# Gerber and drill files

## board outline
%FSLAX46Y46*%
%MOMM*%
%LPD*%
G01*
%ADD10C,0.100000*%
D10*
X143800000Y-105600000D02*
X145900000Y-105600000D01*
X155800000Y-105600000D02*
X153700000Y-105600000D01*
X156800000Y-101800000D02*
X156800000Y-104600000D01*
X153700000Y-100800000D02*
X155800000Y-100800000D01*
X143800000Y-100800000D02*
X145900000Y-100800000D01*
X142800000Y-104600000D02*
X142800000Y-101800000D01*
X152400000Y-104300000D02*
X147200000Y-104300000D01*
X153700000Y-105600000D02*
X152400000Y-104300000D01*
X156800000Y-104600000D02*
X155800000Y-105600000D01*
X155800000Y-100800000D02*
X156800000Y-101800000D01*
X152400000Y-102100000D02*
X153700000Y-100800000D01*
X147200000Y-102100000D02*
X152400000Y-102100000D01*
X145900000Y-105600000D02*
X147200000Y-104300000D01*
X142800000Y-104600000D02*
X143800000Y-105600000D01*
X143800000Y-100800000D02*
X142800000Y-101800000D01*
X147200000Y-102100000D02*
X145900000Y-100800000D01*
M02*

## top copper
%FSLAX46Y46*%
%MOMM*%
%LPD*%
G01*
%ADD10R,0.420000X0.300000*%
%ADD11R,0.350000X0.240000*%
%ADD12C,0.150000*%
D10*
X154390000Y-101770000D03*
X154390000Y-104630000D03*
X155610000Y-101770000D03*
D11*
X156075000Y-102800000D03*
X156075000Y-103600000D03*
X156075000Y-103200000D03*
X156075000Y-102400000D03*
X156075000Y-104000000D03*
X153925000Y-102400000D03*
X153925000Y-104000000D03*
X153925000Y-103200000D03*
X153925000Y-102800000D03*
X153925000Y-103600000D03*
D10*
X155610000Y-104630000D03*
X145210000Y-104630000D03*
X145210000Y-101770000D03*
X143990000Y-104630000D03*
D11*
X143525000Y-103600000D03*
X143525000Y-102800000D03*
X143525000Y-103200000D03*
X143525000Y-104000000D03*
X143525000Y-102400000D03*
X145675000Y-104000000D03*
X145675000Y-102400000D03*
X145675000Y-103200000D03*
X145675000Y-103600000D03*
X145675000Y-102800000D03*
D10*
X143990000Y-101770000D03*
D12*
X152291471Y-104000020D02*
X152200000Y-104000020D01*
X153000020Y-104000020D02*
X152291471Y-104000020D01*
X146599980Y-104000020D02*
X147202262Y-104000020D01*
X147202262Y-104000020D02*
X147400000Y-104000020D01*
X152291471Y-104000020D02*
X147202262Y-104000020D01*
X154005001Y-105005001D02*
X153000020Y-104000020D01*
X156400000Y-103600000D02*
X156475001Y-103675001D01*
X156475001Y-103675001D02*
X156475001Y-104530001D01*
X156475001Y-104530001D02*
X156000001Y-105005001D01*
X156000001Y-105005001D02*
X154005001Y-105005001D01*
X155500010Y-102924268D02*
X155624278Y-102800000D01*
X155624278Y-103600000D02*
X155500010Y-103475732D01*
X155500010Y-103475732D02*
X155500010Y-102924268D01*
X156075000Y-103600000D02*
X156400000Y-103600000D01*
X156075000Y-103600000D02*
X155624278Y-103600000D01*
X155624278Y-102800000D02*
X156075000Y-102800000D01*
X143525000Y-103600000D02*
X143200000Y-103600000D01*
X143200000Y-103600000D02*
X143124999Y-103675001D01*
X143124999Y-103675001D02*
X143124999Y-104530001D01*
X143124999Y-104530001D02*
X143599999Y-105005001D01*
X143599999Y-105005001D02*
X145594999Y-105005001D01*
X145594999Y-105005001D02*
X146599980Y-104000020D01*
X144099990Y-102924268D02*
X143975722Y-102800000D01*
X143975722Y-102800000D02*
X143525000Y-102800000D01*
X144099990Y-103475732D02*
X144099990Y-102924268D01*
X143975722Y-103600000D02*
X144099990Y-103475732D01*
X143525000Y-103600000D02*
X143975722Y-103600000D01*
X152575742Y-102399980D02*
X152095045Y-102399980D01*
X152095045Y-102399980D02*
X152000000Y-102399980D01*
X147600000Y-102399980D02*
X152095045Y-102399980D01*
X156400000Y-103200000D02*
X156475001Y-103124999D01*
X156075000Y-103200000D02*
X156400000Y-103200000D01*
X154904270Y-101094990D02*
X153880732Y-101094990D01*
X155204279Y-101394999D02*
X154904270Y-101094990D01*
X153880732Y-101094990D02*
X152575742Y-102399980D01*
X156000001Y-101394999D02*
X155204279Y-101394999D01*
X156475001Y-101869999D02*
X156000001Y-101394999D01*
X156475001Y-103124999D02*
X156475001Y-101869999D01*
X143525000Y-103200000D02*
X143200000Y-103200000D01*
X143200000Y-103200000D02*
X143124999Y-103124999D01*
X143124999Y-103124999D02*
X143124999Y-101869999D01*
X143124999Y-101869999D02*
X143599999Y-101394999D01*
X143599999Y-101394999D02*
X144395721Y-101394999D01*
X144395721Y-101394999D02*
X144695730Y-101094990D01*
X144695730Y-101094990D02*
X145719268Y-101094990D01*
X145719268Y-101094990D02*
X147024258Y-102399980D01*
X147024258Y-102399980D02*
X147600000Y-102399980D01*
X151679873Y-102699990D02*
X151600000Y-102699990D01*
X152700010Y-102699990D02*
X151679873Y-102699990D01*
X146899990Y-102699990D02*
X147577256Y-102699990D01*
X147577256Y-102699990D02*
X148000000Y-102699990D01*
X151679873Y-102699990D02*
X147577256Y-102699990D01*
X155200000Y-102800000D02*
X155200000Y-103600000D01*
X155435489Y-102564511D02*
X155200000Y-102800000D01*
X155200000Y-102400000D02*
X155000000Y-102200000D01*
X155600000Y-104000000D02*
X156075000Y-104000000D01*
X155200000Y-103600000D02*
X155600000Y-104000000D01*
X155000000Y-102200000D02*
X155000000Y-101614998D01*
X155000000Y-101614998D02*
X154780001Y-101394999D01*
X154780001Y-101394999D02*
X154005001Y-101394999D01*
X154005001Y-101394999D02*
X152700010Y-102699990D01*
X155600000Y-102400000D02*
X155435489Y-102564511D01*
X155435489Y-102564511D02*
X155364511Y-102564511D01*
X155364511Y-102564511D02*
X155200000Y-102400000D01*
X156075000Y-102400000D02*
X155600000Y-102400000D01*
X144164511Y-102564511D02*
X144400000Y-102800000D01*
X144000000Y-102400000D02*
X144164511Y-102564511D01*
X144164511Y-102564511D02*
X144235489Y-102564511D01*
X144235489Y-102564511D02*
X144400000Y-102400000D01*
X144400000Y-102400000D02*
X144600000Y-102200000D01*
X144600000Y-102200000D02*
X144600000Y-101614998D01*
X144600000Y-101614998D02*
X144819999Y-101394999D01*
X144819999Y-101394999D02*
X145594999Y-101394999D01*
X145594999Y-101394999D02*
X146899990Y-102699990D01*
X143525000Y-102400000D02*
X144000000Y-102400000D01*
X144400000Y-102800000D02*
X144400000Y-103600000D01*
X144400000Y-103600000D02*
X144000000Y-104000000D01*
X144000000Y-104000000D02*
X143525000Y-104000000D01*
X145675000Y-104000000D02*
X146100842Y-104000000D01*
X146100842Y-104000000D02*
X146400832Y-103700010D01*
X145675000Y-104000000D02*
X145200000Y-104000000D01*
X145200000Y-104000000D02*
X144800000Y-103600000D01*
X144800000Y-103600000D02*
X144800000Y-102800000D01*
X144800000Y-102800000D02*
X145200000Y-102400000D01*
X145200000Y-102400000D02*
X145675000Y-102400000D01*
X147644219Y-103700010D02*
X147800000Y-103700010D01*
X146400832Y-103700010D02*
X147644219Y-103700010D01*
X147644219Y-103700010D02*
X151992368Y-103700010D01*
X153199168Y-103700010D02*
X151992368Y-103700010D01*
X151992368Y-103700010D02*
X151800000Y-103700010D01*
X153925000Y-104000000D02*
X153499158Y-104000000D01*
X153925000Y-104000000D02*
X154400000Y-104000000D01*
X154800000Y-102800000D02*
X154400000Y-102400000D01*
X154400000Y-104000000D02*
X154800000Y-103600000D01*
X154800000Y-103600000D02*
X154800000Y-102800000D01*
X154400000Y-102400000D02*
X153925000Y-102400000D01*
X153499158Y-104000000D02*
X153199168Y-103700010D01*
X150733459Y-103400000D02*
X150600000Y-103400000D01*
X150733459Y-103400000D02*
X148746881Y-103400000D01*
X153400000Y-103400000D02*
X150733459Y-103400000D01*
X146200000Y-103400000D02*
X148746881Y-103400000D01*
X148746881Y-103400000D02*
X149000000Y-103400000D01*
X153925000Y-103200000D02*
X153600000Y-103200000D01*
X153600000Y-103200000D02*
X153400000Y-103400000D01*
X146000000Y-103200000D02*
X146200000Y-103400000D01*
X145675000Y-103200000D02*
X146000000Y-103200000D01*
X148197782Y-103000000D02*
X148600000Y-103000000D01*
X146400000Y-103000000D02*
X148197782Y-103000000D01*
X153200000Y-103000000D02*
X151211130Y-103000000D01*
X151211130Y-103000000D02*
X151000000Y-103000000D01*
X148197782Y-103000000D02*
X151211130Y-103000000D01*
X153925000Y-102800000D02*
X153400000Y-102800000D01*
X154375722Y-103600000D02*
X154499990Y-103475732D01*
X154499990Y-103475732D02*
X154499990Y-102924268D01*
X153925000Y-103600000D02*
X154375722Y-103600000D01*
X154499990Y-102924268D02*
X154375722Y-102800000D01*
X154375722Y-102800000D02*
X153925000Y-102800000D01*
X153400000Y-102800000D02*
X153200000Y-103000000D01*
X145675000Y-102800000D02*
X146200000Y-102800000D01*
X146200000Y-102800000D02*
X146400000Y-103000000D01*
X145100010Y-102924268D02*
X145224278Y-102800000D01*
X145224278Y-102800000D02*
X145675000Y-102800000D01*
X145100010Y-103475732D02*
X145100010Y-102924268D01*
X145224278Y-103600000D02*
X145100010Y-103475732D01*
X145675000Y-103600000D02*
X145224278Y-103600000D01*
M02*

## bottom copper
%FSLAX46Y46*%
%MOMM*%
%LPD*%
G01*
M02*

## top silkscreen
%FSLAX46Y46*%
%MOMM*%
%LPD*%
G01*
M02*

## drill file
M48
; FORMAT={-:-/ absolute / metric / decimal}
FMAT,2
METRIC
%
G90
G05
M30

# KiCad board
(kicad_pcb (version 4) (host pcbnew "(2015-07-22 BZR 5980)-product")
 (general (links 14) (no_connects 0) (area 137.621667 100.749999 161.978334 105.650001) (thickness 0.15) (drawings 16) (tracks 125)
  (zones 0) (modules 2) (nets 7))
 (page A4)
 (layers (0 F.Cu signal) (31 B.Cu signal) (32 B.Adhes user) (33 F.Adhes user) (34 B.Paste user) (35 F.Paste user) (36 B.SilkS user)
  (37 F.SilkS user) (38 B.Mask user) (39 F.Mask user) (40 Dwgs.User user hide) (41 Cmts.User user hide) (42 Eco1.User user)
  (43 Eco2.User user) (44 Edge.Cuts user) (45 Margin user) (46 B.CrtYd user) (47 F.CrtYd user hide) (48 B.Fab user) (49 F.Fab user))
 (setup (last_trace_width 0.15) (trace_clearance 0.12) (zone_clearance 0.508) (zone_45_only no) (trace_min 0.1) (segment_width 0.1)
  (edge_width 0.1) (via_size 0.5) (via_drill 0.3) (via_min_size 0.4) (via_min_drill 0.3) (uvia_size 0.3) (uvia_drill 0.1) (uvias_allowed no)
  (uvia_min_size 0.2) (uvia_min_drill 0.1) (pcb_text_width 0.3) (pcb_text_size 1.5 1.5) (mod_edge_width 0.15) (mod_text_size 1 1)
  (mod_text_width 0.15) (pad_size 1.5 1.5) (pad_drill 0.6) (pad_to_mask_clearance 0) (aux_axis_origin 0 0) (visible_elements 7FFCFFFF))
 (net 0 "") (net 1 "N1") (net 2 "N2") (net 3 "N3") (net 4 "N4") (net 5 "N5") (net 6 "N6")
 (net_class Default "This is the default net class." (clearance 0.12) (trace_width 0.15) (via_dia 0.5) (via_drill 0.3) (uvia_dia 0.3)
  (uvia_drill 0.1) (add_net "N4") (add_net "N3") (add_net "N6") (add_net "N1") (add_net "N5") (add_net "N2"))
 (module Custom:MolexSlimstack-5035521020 (layer F.Cu) (at 155 103.2 270)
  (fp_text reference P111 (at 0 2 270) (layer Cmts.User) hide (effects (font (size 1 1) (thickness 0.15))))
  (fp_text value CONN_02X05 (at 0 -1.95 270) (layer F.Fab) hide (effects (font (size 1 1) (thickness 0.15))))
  (pad "" smd rect (at 0.8 -0.65 90) (size 0.3 0.5) (layers Dwgs.User))
  (pad "" smd rect (at 0 -0.65 90) (size 0.3 0.5) (layers Dwgs.User))
  (pad "" smd rect (at -0.4 -0.65 90) (size 0.3 0.5) (layers Dwgs.User))
  (pad "" smd rect (at -0.8 -0.65 90) (size 0.3 0.5) (layers Dwgs.User))
  (pad "" smd rect (at 0.4 -0.65 90) (size 0.3 0.5) (layers Dwgs.User))
  (pad "" smd rect (at -0.8 0.65 270) (size 0.3 0.5) (layers Dwgs.User))
  (pad "" smd rect (at -0.4 0.65 270) (size 0.3 0.5) (layers Dwgs.User))
  (pad "" smd rect (at 0.8 0.65 270) (size 0.3 0.5) (layers Dwgs.User))
  (pad "" smd rect (at 0.4 0.65 270) (size 0.3 0.5) (layers Dwgs.User))
  (pad "" smd rect (at -1.43 0.61 90) (size 0.3 0.42) (layers F.Cu F.Paste F.Mask))
  (pad "" smd rect (at 1.43 0.61 270) (size 0.3 0.42) (layers F.Cu F.Paste F.Mask))
  (pad "" smd rect (at -1.43 -0.61 90) (size 0.3 0.42) (layers F.Cu F.Paste F.Mask))
  (pad 4 smd rect (at -0.4 -1.075 270) (size 0.24 0.35) (layers F.Cu F.Paste F.Mask) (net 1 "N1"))
  (pad 8 smd rect (at 0.4 -1.075 270) (size 0.24 0.35) (layers F.Cu F.Paste F.Mask) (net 1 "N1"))
  (pad 6 smd rect (at 0 -1.075 270) (size 0.24 0.35) (layers F.Cu F.Paste F.Mask) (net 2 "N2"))
  (pad 2 smd rect (at -0.8 -1.075 270) (size 0.24 0.35) (layers F.Cu F.Paste F.Mask) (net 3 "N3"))
  (pad 10 smd rect (at 0.8 -1.075 270) (size 0.24 0.35) (layers F.Cu F.Paste F.Mask) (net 3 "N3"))
  (pad 1 smd rect (at -0.8 1.075 90) (size 0.24 0.35) (layers F.Cu F.Paste F.Mask) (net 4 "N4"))
  (pad 9 smd rect (at 0.8 1.075 90) (size 0.24 0.35) (layers F.Cu F.Paste F.Mask) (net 4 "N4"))
  (pad 5 smd rect (at 0 1.075 90) (size 0.24 0.35) (layers F.Cu F.Paste F.Mask) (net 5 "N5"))
  (pad 3 smd rect (at -0.4 1.075 90) (size 0.24 0.35) (layers F.Cu F.Paste F.Mask) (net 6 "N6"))
  (pad 7 smd rect (at 0.4 1.075 90) (size 0.24 0.35) (layers F.Cu F.Paste F.Mask) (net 6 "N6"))
  (pad "" smd rect (at 1.43 -0.61 270) (size 0.3 0.42) (layers F.Cu F.Paste F.Mask))
  (pad "" smd rect (at 0 0.65 270) (size 0.3 0.5) (layers Dwgs.User)))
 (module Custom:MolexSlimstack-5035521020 (layer F.Cu) (at 144.6 103.2 90)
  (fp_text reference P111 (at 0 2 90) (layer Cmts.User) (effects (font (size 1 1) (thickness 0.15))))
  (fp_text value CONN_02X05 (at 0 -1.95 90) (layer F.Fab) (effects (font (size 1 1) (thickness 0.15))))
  (pad "" smd rect (at 0.8 -0.65 270) (size 0.3 0.5) (layers Dwgs.User))
  (pad "" smd rect (at 0 -0.65 270) (size 0.3 0.5) (layers Dwgs.User))
  (pad "" smd rect (at -0.4 -0.65 270) (size 0.3 0.5) (layers Dwgs.User))
  (pad "" smd rect (at -0.8 -0.65 270) (size 0.3 0.5) (layers Dwgs.User))
  (pad "" smd rect (at 0.4 -0.65 270) (size 0.3 0.5) (layers Dwgs.User))
  (pad "" smd rect (at -0.8 0.65 90) (size 0.3 0.5) (layers Dwgs.User))
  (pad "" smd rect (at -0.4 0.65 90) (size 0.3 0.5) (layers Dwgs.User))
  (pad "" smd rect (at 0.8 0.65 90) (size 0.3 0.5) (layers Dwgs.User))
  (pad "" smd rect (at 0.4 0.65 90) (size 0.3 0.5) (layers Dwgs.User))
  (pad "" smd rect (at -1.43 0.61 270) (size 0.3 0.42) (layers F.Cu F.Paste F.Mask))
  (pad "" smd rect (at 1.43 0.61 90) (size 0.3 0.42) (layers F.Cu F.Paste F.Mask))
  (pad "" smd rect (at -1.43 -0.61 270) (size 0.3 0.42) (layers F.Cu F.Paste F.Mask))
  (pad 4 smd rect (at -0.4 -1.075 90) (size 0.24 0.35) (layers F.Cu F.Paste F.Mask) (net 1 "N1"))
  (pad 8 smd rect (at 0.4 -1.075 90) (size 0.24 0.35) (layers F.Cu F.Paste F.Mask) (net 1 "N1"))
  (pad 6 smd rect (at 0 -1.075 90) (size 0.24 0.35) (layers F.Cu F.Paste F.Mask) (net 2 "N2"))
  (pad 2 smd rect (at -0.8 -1.075 90) (size 0.24 0.35) (layers F.Cu F.Paste F.Mask) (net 3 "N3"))
  (pad 10 smd rect (at 0.8 -1.075 90) (size 0.24 0.35) (layers F.Cu F.Paste F.Mask) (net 3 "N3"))
  (pad 1 smd rect (at -0.8 1.075 270) (size 0.24 0.35) (layers F.Cu F.Paste F.Mask) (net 4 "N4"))
  (pad 9 smd rect (at 0.8 1.075 270) (size 0.24 0.35) (layers F.Cu F.Paste F.Mask) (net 4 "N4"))
  (pad 5 smd rect (at 0 1.075 270) (size 0.24 0.35) (layers F.Cu F.Paste F.Mask) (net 5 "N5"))
  (pad 3 smd rect (at -0.4 1.075 270) (size 0.24 0.35) (layers F.Cu F.Paste F.Mask) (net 6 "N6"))
  (pad 7 smd rect (at 0.4 1.075 270) (size 0.24 0.35) (layers F.Cu F.Paste F.Mask) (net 6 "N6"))
  (pad "" smd rect (at 1.43 -0.61 90) (size 0.3 0.42) (layers F.Cu F.Paste F.Mask))
  (pad "" smd rect (at 0 0.65 90) (size 0.3 0.5) (layers Dwgs.User)))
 (gr_line (start 143.8 105.6) (end 145.9 105.6) (layer Edge.Cuts) (width 0.1))
 (gr_line (start 155.8 105.6) (end 153.7 105.6) (layer Edge.Cuts) (width 0.1))
 (gr_line (start 156.8 101.8) (end 156.8 104.6) (layer Edge.Cuts) (width 0.1))
 (gr_line (start 153.7 100.8) (end 155.8 100.8) (layer Edge.Cuts) (width 0.1))
 (gr_line (start 143.8 100.8) (end 145.9 100.8) (layer Edge.Cuts) (width 0.1))
 (gr_line (start 142.8 104.6) (end 142.8 101.8) (layer Edge.Cuts) (width 0.1))
 (gr_line (start 152.4 104.3) (end 147.2 104.3) (layer Edge.Cuts) (width 0.1))
 (gr_line (start 153.7 105.6) (end 152.4 104.3) (layer Edge.Cuts) (width 0.1))
 (gr_line (start 156.8 104.6) (end 155.8 105.6) (layer Edge.Cuts) (width 0.1))
 (gr_line (start 155.8 100.8) (end 156.8 101.8) (layer Edge.Cuts) (width 0.1))
 (gr_line (start 152.4 102.1) (end 153.7 100.8) (layer Edge.Cuts) (width 0.1))
 (gr_line (start 147.2 102.1) (end 152.4 102.1) (layer Edge.Cuts) (width 0.1))
 (gr_line (start 145.9 105.6) (end 147.2 104.3) (layer Edge.Cuts) (width 0.1))
 (gr_line (start 142.8 104.6) (end 143.8 105.6) (layer Edge.Cuts) (width 0.1))
 (gr_line (start 143.8 100.8) (end 142.8 101.8) (layer Edge.Cuts) (width 0.1))
 (gr_line (start 147.2 102.1) (end 145.9 100.8) (layer Edge.Cuts) (width 0.1))
 (segment (start 152.291471 104.00002) (end 152.2 104.00002) (width 0.15) (layer F.Cu) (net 1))
 (segment (start 153.00002 104.00002) (end 152.291471 104.00002) (width 0.15) (layer F.Cu) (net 1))
 (segment (start 146.59998 104.00002) (end 147.202262 104.00002) (width 0.15) (layer F.Cu) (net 1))
 (segment (start 147.202262 104.00002) (end 147.4 104.00002) (width 0.15) (layer F.Cu) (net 1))
 (segment (start 152.291471 104.00002) (end 147.202262 104.00002) (width 0.15) (layer F.Cu) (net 1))
 (segment (start 154.005001 105.005001) (end 153.00002 104.00002) (width 0.15) (layer F.Cu) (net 1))
 (segment (start 156.4 103.6) (end 156.475001 103.675001) (width 0.15) (layer F.Cu) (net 1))
 (segment (start 156.475001 103.675001) (end 156.475001 104.530001) (width 0.15) (layer F.Cu) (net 1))
 (segment (start 156.475001 104.530001) (end 156.000001 105.005001) (width 0.15) (layer F.Cu) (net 1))
 (segment (start 156.000001 105.005001) (end 154.005001 105.005001) (width 0.15) (layer F.Cu) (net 1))
 (segment (start 155.50001 102.924268) (end 155.624278 102.8) (width 0.15) (layer F.Cu) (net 1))
 (segment (start 155.624278 103.6) (end 155.50001 103.475732) (width 0.15) (layer F.Cu) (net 1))
 (segment (start 155.50001 103.475732) (end 155.50001 102.924268) (width 0.15) (layer F.Cu) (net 1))
 (segment (start 156.075 103.6) (end 156.4 103.6) (width 0.15) (layer F.Cu) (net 1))
 (segment (start 156.075 103.6) (end 155.624278 103.6) (width 0.15) (layer F.Cu) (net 1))
 (segment (start 155.624278 102.8) (end 156.075 102.8) (width 0.15) (layer F.Cu) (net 1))
 (segment (start 143.525 103.6) (end 143.2 103.6) (width 0.15) (layer F.Cu) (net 1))
 (segment (start 143.2 103.6) (end 143.124999 103.675001) (width 0.15) (layer F.Cu) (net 1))
 (segment (start 143.124999 103.675001) (end 143.124999 104.530001) (width 0.15) (layer F.Cu) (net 1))
 (segment (start 143.124999 104.530001) (end 143.599999 105.005001) (width 0.15) (layer F.Cu) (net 1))
 (segment (start 143.599999 105.005001) (end 145.594999 105.005001) (width 0.15) (layer F.Cu) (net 1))
 (segment (start 145.594999 105.005001) (end 146.59998 104.00002) (width 0.15) (layer F.Cu) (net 1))
 (segment (start 144.09999 102.924268) (end 143.975722 102.8) (width 0.15) (layer F.Cu) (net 1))
 (segment (start 143.975722 102.8) (end 143.525 102.8) (width 0.15) (layer F.Cu) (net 1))
 (segment (start 144.09999 103.475732) (end 144.09999 102.924268) (width 0.15) (layer F.Cu) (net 1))
 (segment (start 143.975722 103.6) (end 144.09999 103.475732) (width 0.15) (layer F.Cu) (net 1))
 (segment (start 143.525 103.6) (end 143.975722 103.6) (width 0.15) (layer F.Cu) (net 1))
 (segment (start 152.575742 102.39998) (end 152.095045 102.39998) (width 0.15) (layer F.Cu) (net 2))
 (segment (start 152.095045 102.39998) (end 152 102.39998) (width 0.15) (layer F.Cu) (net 2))
 (segment (start 147.6 102.39998) (end 152.095045 102.39998) (width 0.15) (layer F.Cu) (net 2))
 (segment (start 156.4 103.2) (end 156.475001 103.124999) (width 0.15) (layer F.Cu) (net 2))
 (segment (start 156.075 103.2) (end 156.4 103.2) (width 0.15) (layer F.Cu) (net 2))
 (segment (start 154.90427 101.09499) (end 153.880732 101.09499) (width 0.15) (layer F.Cu) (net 2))
 (segment (start 155.204279 101.394999) (end 154.90427 101.09499) (width 0.15) (layer F.Cu) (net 2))
 (segment (start 153.880732 101.09499) (end 152.575742 102.39998) (width 0.15) (layer F.Cu) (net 2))
 (segment (start 156.000001 101.394999) (end 155.204279 101.394999) (width 0.15) (layer F.Cu) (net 2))
 (segment (start 156.475001 101.869999) (end 156.000001 101.394999) (width 0.15) (layer F.Cu) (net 2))
 (segment (start 156.475001 103.124999) (end 156.475001 101.869999) (width 0.15) (layer F.Cu) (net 2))
 (segment (start 143.525 103.2) (end 143.2 103.2) (width 0.15) (layer F.Cu) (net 2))
 (segment (start 143.2 103.2) (end 143.124999 103.124999) (width 0.15) (layer F.Cu) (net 2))
 (segment (start 143.124999 103.124999) (end 143.124999 101.869999) (width 0.15) (layer F.Cu) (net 2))
 (segment (start 143.124999 101.869999) (end 143.599999 101.394999) (width 0.15) (layer F.Cu) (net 2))
 (segment (start 143.599999 101.394999) (end 144.395721 101.394999) (width 0.15) (layer F.Cu) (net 2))
 (segment (start 144.395721 101.394999) (end 144.69573 101.09499) (width 0.15) (layer F.Cu) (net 2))
 (segment (start 144.69573 101.09499) (end 145.719268 101.09499) (width 0.15) (layer F.Cu) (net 2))
 (segment (start 145.719268 101.09499) (end 147.024258 102.39998) (width 0.15) (layer F.Cu) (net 2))
 (segment (start 147.024258 102.39998) (end 147.6 102.39998) (width 0.15) (layer F.Cu) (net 2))
 (segment (start 151.679873 102.69999) (end 151.6 102.69999) (width 0.15) (layer F.Cu) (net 3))
 (segment (start 152.70001 102.69999) (end 151.679873 102.69999) (width 0.15) (layer F.Cu) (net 3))
 (segment (start 146.89999 102.69999) (end 147.577256 102.69999) (width 0.15) (layer F.Cu) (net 3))
 (segment (start 147.577256 102.69999) (end 148 102.69999) (width 0.15) (layer F.Cu) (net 3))
 (segment (start 151.679873 102.69999) (end 147.577256 102.69999) (width 0.15) (layer F.Cu) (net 3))
 (segment (start 155.2 102.8) (end 155.2 103.6) (width 0.15) (layer F.Cu) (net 3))
 (segment (start 155.435489 102.564511) (end 155.2 102.8) (width 0.15) (layer F.Cu) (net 3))
 (segment (start 155.2 102.4) (end 155 102.2) (width 0.15) (layer F.Cu) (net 3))
 (segment (start 155.6 104) (end 156.075 104) (width 0.15) (layer F.Cu) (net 3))
 (segment (start 155.2 103.6) (end 155.6 104) (width 0.15) (layer F.Cu) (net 3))
 (segment (start 155 102.2) (end 155 101.614998) (width 0.15) (layer F.Cu) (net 3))
 (segment (start 155 101.614998) (end 154.780001 101.394999) (width 0.15) (layer F.Cu) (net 3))
 (segment (start 154.780001 101.394999) (end 154.005001 101.394999) (width 0.15) (layer F.Cu) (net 3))
 (segment (start 154.005001 101.394999) (end 152.70001 102.69999) (width 0.15) (layer F.Cu) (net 3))
 (segment (start 155.6 102.4) (end 155.435489 102.564511) (width 0.15) (layer F.Cu) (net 3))
 (segment (start 155.435489 102.564511) (end 155.364511 102.564511) (width 0.15) (layer F.Cu) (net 3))
 (segment (start 155.364511 102.564511) (end 155.2 102.4) (width 0.15) (layer F.Cu) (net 3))
 (segment (start 156.075 102.4) (end 155.6 102.4) (width 0.15) (layer F.Cu) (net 3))
 (segment (start 144.164511 102.564511) (end 144.4 102.8) (width 0.15) (layer F.Cu) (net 3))
 (segment (start 144 102.4) (end 144.164511 102.564511) (width 0.15) (layer F.Cu) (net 3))
 (segment (start 144.164511 102.564511) (end 144.235489 102.564511) (width 0.15) (layer F.Cu) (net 3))
 (segment (start 144.235489 102.564511) (end 144.4 102.4) (width 0.15) (layer F.Cu) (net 3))
 (segment (start 144.4 102.4) (end 144.6 102.2) (width 0.15) (layer F.Cu) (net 3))
 (segment (start 144.6 102.2) (end 144.6 101.614998) (width 0.15) (layer F.Cu) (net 3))
 (segment (start 144.6 101.614998) (end 144.819999 101.394999) (width 0.15) (layer F.Cu) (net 3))
 (segment (start 144.819999 101.394999) (end 145.594999 101.394999) (width 0.15) (layer F.Cu) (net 3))
 (segment (start 145.594999 101.394999) (end 146.89999 102.69999) (width 0.15) (layer F.Cu) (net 3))
 (segment (start 143.525 102.4) (end 144 102.4) (width 0.15) (layer F.Cu) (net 3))
 (segment (start 144.4 102.8) (end 144.4 103.6) (width 0.15) (layer F.Cu) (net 3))
 (segment (start 144.4 103.6) (end 144 104) (width 0.15) (layer F.Cu) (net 3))
 (segment (start 144 104) (end 143.525 104) (width 0.15) (layer F.Cu) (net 3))
 (segment (start 145.675 104) (end 146.100842 104) (width 0.15) (layer F.Cu) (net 4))
 (segment (start 146.100842 104) (end 146.400832 103.70001) (width 0.15) (layer F.Cu) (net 4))
 (segment (start 145.675 104) (end 145.2 104) (width 0.15) (layer F.Cu) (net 4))
 (segment (start 145.2 104) (end 144.8 103.6) (width 0.15) (layer F.Cu) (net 4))
 (segment (start 144.8 103.6) (end 144.8 102.8) (width 0.15) (layer F.Cu) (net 4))
 (segment (start 144.8 102.8) (end 145.2 102.4) (width 0.15) (layer F.Cu) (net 4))
 (segment (start 145.2 102.4) (end 145.675 102.4) (width 0.15) (layer F.Cu) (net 4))
 (segment (start 147.644219 103.70001) (end 147.8 103.70001) (width 0.15) (layer F.Cu) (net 4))
 (segment (start 146.400832 103.70001) (end 147.644219 103.70001) (width 0.15) (layer F.Cu) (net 4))
 (segment (start 147.644219 103.70001) (end 151.992368 103.70001) (width 0.15) (layer F.Cu) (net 4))
 (segment (start 153.199168 103.70001) (end 151.992368 103.70001) (width 0.15) (layer F.Cu) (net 4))
 (segment (start 151.992368 103.70001) (end 151.8 103.70001) (width 0.15) (layer F.Cu) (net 4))
 (segment (start 153.925 104) (end 153.499158 104) (width 0.15) (layer F.Cu) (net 4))
 (segment (start 153.925 104) (end 154.4 104) (width 0.15) (layer F.Cu) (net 4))
 (segment (start 154.8 102.8) (end 154.4 102.4) (width 0.15) (layer F.Cu) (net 4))
 (segment (start 154.4 104) (end 154.8 103.6) (width 0.15) (layer F.Cu) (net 4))
 (segment (start 154.8 103.6) (end 154.8 102.8) (width 0.15) (layer F.Cu) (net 4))
 (segment (start 154.4 102.4) (end 153.925 102.4) (width 0.15) (layer F.Cu) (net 4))
 (segment (start 153.499158 104) (end 153.199168 103.70001) (width 0.15) (layer F.Cu) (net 4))
 (segment (start 150.733459 103.4) (end 150.6 103.4) (width 0.15) (layer F.Cu) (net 5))
 (segment (start 150.733459 103.4) (end 148.746881 103.4) (width 0.15) (layer F.Cu) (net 5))
 (segment (start 153.4 103.4) (end 150.733459 103.4) (width 0.15) (layer F.Cu) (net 5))
 (segment (start 146.2 103.4) (end 148.746881 103.4) (width 0.15) (layer F.Cu) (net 5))
 (segment (start 148.746881 103.4) (end 149 103.4) (width 0.15) (layer F.Cu) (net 5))
 (segment (start 153.925 103.2) (end 153.6 103.2) (width 0.15) (layer F.Cu) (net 5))
 (segment (start 153.6 103.2) (end 153.4 103.4) (width 0.15) (layer F.Cu) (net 5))
 (segment (start 146 103.2) (end 146.2 103.4) (width 0.15) (layer F.Cu) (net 5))
 (segment (start 145.675 103.2) (end 146 103.2) (width 0.15) (layer F.Cu) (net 5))
 (segment (start 148.197782 103) (end 148.6 103) (width 0.15) (layer F.Cu) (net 6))
 (segment (start 146.4 103) (end 148.197782 103) (width 0.15) (layer F.Cu) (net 6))
 (segment (start 153.2 103) (end 151.21113 103) (width 0.15) (layer F.Cu) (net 6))
 (segment (start 151.21113 103) (end 151 103) (width 0.15) (layer F.Cu) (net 6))
 (segment (start 148.197782 103) (end 151.21113 103) (width 0.15) (layer F.Cu) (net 6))
 (segment (start 153.925 102.8) (end 153.4 102.8) (width 0.15) (layer F.Cu) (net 6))
 (segment (start 154.375722 103.6) (end 154.49999 103.475732) (width 0.15) (layer F.Cu) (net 6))
 (segment (start 154.49999 103.475732) (end 154.49999 102.924268) (width 0.15) (layer F.Cu) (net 6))
 (segment (start 153.925 103.6) (end 154.375722 103.6) (width 0.15) (layer F.Cu) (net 6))
 (segment (start 154.49999 102.924268) (end 154.375722 102.8) (width 0.15) (layer F.Cu) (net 6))
 (segment (start 154.375722 102.8) (end 153.925 102.8) (width 0.15) (layer F.Cu) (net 6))
 (segment (start 153.4 102.8) (end 153.2 103) (width 0.15) (layer F.Cu) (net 6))
 (segment (start 145.675 102.8) (end 146.2 102.8) (width 0.15) (layer F.Cu) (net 6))
 (segment (start 146.2 102.8) (end 146.4 103) (width 0.15) (layer F.Cu) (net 6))
 (segment (start 145.10001 102.924268) (end 145.224278 102.8) (width 0.15) (layer F.Cu) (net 6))
 (segment (start 145.224278 102.8) (end 145.675 102.8) (width 0.15) (layer F.Cu) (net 6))
 (segment (start 145.10001 103.475732) (end 145.10001 102.924268) (width 0.15) (layer F.Cu) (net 6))
 (segment (start 145.224278 103.6) (end 145.10001 103.475732) (width 0.15) (layer F.Cu) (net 6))
 (segment (start 145.675 103.6) (end 145.224278 103.6) (width 0.15) (layer F.Cu) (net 6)))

